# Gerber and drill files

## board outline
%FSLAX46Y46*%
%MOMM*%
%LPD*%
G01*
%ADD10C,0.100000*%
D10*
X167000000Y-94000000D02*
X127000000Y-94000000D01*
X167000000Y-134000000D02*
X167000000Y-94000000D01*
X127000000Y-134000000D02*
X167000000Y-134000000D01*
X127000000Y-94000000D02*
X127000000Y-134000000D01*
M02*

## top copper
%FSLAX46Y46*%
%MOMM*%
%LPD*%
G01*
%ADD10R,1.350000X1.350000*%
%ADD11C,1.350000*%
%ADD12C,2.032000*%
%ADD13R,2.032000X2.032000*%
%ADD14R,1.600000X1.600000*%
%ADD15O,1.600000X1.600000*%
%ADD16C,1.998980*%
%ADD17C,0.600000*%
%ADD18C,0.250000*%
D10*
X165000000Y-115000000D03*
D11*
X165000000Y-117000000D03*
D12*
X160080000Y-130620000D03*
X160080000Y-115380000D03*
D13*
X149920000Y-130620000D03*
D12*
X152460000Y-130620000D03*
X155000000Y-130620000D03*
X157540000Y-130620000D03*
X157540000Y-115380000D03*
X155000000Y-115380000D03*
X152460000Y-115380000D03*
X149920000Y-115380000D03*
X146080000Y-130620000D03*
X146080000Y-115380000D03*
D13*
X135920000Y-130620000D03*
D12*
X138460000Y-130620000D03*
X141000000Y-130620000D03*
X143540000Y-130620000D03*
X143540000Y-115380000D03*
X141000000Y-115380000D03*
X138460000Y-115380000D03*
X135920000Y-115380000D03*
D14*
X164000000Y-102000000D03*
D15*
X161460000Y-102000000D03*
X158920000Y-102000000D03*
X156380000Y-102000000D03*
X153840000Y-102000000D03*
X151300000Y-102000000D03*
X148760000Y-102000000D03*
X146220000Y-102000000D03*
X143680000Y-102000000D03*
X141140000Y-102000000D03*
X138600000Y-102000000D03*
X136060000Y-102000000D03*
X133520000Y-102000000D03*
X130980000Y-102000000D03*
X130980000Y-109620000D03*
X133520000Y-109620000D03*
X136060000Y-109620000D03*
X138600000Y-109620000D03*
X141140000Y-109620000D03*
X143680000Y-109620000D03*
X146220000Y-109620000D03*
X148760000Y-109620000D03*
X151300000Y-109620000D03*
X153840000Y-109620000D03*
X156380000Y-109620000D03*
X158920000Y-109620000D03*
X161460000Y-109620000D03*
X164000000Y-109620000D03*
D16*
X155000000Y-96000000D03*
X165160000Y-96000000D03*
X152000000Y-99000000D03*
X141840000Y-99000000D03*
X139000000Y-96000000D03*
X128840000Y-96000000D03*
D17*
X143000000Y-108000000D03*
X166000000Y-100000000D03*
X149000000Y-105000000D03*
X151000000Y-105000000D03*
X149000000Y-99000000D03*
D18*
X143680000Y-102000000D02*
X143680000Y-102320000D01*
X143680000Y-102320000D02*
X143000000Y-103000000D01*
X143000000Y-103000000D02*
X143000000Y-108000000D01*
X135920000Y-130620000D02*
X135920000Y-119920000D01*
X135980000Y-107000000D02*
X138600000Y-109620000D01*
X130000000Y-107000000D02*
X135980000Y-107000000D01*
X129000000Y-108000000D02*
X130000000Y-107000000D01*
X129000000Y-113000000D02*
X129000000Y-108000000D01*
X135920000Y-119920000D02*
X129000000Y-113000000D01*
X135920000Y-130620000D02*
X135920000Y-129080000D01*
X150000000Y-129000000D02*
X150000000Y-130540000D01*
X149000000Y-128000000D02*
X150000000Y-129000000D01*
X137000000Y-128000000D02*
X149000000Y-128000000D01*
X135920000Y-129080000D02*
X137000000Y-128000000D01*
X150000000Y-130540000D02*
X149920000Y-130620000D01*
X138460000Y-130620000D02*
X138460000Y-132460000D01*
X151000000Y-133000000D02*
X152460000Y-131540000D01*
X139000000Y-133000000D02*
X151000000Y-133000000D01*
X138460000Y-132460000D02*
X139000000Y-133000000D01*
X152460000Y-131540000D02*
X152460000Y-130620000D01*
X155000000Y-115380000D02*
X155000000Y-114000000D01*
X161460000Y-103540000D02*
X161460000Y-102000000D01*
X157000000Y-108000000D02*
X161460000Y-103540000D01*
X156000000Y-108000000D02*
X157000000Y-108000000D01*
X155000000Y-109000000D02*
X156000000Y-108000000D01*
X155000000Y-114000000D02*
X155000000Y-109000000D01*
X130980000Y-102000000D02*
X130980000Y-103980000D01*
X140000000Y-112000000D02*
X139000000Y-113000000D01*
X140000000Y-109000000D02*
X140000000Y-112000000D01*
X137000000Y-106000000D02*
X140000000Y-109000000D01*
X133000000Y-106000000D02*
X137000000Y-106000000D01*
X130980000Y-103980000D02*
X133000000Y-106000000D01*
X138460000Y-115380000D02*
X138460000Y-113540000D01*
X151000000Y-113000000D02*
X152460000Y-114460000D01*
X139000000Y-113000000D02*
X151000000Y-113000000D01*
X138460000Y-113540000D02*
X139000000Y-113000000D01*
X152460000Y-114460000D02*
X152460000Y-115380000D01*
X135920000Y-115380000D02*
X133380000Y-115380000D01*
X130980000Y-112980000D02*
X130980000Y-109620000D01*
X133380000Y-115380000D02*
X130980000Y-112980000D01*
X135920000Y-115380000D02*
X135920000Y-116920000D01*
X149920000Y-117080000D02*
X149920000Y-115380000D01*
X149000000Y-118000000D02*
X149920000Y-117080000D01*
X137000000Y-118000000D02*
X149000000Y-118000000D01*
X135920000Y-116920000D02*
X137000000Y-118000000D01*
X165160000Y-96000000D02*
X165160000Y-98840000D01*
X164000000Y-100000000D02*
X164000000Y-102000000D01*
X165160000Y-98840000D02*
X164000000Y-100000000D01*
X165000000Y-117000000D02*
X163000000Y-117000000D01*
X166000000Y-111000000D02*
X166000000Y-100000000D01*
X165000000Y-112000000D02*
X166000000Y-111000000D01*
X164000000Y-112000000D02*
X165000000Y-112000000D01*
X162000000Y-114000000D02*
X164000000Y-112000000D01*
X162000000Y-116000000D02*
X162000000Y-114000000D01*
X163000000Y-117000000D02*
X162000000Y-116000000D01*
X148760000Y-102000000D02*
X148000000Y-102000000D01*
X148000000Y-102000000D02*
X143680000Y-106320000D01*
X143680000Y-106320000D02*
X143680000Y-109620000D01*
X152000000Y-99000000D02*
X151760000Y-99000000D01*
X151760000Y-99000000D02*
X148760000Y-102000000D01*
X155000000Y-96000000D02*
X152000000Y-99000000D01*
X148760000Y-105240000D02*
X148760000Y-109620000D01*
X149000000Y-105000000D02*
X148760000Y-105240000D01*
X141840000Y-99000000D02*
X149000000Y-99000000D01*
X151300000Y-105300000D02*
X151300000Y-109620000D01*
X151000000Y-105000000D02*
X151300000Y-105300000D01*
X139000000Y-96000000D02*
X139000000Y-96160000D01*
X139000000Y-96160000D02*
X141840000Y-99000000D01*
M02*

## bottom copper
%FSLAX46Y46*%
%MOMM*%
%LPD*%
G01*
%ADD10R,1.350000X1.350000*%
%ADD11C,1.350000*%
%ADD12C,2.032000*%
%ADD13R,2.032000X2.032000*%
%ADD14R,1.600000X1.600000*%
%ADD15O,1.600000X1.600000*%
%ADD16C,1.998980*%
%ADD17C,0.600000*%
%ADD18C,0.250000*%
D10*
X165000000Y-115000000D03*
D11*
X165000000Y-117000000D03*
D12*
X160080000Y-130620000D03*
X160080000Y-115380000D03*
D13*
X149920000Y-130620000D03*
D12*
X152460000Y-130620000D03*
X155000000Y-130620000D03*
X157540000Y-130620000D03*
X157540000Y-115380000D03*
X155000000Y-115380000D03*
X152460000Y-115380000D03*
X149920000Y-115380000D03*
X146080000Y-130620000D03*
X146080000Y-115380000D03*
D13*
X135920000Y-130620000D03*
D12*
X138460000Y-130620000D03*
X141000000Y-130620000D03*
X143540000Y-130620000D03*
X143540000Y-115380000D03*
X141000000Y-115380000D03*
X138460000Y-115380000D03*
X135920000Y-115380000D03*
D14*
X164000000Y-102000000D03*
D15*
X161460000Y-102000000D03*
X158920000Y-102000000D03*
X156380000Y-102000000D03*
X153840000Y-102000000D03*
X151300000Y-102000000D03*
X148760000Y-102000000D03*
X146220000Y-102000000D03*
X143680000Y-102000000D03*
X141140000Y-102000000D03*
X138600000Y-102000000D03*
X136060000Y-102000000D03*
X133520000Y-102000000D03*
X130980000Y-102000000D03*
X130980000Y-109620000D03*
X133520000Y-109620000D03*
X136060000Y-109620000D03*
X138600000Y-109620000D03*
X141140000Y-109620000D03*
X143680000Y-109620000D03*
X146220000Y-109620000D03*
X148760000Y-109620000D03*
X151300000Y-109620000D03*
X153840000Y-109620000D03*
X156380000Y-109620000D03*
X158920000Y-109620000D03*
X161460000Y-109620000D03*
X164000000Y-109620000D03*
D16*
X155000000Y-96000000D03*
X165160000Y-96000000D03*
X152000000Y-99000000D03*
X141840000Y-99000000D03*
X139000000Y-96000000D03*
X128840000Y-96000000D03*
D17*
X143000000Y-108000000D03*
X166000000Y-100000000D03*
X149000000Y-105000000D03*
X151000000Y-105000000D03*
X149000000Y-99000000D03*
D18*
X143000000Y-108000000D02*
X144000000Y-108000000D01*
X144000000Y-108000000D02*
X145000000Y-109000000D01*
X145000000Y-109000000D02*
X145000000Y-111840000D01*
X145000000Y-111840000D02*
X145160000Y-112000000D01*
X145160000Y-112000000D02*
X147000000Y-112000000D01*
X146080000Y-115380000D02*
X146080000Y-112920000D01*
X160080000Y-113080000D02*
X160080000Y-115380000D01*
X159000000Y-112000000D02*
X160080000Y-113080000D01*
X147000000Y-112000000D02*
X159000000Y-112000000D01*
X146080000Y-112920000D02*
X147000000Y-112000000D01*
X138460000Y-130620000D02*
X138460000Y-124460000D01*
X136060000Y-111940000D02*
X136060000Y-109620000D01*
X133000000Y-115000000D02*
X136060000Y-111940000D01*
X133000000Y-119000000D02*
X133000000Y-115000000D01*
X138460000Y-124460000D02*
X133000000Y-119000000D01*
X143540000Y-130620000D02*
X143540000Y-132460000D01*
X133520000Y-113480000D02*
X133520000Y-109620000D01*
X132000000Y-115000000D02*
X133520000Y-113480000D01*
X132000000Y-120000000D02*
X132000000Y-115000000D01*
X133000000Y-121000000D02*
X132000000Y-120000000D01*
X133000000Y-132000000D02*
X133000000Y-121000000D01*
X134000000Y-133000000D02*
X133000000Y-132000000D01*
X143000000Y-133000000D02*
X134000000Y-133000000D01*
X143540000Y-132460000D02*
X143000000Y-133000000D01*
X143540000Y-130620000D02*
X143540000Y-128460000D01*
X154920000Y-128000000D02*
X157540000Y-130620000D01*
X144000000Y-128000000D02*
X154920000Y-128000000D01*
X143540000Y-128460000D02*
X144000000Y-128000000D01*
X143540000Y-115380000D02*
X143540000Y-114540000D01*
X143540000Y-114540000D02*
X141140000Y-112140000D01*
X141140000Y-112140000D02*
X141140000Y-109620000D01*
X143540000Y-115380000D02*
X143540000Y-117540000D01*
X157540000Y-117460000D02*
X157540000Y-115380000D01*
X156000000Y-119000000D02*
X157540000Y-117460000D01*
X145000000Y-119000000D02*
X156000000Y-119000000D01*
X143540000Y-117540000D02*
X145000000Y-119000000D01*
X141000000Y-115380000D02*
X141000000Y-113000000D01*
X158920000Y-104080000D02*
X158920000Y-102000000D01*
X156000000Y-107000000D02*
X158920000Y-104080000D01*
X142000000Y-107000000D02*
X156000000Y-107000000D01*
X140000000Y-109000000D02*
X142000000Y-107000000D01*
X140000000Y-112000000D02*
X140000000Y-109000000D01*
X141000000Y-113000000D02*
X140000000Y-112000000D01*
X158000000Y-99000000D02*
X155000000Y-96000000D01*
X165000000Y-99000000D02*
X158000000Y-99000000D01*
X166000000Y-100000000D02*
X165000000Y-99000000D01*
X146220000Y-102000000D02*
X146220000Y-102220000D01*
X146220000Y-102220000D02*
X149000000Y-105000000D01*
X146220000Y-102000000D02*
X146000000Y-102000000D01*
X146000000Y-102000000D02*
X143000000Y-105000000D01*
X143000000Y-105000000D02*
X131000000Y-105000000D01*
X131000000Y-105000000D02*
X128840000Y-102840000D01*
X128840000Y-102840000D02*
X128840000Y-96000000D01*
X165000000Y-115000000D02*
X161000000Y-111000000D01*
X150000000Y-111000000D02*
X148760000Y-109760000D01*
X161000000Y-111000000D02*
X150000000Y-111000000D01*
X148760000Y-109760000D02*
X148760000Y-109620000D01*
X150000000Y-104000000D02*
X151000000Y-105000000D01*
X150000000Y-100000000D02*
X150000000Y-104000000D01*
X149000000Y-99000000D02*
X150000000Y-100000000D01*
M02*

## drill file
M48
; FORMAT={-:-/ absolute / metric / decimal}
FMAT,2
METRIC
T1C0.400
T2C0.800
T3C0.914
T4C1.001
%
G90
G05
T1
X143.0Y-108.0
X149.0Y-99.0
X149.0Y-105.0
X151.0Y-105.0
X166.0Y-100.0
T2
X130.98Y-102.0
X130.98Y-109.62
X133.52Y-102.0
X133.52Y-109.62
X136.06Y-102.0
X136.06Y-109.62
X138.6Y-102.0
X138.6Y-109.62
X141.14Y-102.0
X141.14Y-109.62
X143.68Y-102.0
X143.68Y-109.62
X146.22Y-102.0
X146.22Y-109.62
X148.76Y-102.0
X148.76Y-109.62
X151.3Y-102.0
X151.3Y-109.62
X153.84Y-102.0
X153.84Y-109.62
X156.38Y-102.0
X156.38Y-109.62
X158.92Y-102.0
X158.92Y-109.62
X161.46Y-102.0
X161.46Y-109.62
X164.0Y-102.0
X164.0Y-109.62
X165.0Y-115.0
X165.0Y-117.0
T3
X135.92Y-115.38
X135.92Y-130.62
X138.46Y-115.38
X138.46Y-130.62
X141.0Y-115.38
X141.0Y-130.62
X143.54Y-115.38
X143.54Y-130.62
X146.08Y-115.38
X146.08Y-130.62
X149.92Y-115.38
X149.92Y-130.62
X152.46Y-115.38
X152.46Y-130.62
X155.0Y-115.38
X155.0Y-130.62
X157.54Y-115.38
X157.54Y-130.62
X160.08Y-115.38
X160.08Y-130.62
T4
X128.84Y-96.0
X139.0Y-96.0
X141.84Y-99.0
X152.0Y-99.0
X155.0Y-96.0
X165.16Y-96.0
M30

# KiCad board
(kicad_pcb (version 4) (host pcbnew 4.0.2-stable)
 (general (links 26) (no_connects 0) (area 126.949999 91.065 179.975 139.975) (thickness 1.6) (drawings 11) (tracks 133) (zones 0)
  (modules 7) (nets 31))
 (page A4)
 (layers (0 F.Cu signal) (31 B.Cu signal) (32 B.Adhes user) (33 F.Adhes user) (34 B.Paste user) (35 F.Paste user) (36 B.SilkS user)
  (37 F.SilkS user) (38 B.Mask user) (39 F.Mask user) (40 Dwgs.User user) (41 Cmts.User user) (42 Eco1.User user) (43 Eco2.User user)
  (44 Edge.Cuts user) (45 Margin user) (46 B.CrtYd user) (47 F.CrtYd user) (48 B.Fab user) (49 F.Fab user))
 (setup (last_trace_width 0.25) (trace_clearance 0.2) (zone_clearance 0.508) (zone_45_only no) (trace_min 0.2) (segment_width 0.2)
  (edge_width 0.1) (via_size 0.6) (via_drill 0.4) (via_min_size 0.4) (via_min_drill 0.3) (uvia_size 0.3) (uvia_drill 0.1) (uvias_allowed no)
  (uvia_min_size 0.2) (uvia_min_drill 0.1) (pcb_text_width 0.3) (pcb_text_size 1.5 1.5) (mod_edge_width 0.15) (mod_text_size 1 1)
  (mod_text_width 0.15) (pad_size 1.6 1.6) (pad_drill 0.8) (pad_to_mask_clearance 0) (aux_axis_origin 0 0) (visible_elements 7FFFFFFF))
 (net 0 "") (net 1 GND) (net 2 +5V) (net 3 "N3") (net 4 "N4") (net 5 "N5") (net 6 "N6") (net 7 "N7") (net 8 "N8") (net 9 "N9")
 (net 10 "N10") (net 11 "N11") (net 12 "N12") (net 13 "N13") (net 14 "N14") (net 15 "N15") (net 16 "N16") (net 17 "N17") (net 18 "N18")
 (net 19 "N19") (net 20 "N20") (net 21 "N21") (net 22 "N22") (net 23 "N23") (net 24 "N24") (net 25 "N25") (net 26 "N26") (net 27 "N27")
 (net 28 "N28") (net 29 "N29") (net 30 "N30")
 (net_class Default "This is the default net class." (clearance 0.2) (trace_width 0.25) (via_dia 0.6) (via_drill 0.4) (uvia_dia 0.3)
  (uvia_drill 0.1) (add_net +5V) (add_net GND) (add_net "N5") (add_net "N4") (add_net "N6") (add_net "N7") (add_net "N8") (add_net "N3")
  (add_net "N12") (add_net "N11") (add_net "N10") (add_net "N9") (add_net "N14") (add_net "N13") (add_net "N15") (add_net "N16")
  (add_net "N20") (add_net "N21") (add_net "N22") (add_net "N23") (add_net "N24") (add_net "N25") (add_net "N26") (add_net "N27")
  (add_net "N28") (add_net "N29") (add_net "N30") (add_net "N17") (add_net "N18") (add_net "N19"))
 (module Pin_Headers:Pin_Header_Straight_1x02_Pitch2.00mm (layer F.Cu) (at 165 115)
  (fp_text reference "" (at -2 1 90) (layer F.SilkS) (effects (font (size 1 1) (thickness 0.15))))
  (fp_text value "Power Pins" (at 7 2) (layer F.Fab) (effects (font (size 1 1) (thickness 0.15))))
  (pad 1 thru_hole rect (at 0 0) (size 1.35 1.35) (drill 0.8) (layers *.Cu *.Mask) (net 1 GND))
  (pad 2 thru_hole circle (at 0 2) (size 1.35 1.35) (drill 0.8) (layers *.Cu *.Mask) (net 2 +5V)))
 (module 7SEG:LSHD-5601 (layer F.Cu) (at 155 123)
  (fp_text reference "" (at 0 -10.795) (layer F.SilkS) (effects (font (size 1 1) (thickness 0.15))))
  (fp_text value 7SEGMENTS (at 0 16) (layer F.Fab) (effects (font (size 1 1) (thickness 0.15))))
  (pad 5 thru_hole circle (at 5.08 7.62) (size 2.032 2.032) (drill 0.9144) (layers *.Cu *.Mask F.SilkS) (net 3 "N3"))
  (pad 10 thru_hole circle (at 5.08 -7.62) (size 2.032 2.032) (drill 0.9144) (layers *.Cu *.Mask F.SilkS) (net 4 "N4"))
  (pad 1 thru_hole rect (at -5.08 7.62) (size 2.032 2.032) (drill 0.9144) (layers *.Cu *.Mask F.SilkS) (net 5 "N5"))
  (pad 2 thru_hole circle (at -2.54 7.62) (size 2.032 2.032) (drill 0.9144) (layers *.Cu *.Mask F.SilkS) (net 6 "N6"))
  (pad 3 thru_hole circle (at 0 7.62) (size 2.032 2.032) (drill 0.9144) (layers *.Cu *.Mask F.SilkS) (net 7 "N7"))
  (pad 4 thru_hole circle (at 2.54 7.62) (size 2.032 2.032) (drill 0.9144) (layers *.Cu *.Mask F.SilkS) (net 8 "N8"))
  (pad 9 thru_hole circle (at 2.54 -7.62) (size 2.032 2.032) (drill 0.9144) (layers *.Cu *.Mask F.SilkS) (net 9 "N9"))
  (pad 8 thru_hole circle (at 0 -7.62) (size 2.032 2.032) (drill 0.9144) (layers *.Cu *.Mask F.SilkS) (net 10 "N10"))
  (pad 7 thru_hole circle (at -2.54 -7.62) (size 2.032 2.032) (drill 0.9144) (layers *.Cu *.Mask F.SilkS) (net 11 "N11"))
  (pad 6 thru_hole circle (at -5.08 -7.62) (size 2.032 2.032) (drill 0.9144) (layers *.Cu *.Mask F.SilkS) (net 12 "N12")))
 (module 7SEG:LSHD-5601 (layer F.Cu) (at 141 123)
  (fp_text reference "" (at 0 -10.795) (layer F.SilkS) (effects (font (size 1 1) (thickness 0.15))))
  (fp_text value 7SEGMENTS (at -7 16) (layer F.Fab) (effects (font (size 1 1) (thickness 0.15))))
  (pad 5 thru_hole circle (at 5.08 7.62) (size 2.032 2.032) (drill 0.9144) (layers *.Cu *.Mask F.SilkS) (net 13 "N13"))
  (pad 10 thru_hole circle (at 5.08 -7.62) (size 2.032 2.032) (drill 0.9144) (layers *.Cu *.Mask F.SilkS) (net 4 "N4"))
  (pad 1 thru_hole rect (at -5.08 7.62) (size 2.032 2.032) (drill 0.9144) (layers *.Cu *.Mask F.SilkS) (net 5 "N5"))
  (pad 2 thru_hole circle (at -2.54 7.62) (size 2.032 2.032) (drill 0.9144) (layers *.Cu *.Mask F.SilkS) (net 6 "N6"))
  (pad 3 thru_hole circle (at 0 7.62) (size 2.032 2.032) (drill 0.9144) (layers *.Cu *.Mask F.SilkS) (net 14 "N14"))
  (pad 4 thru_hole circle (at 2.54 7.62) (size 2.032 2.032) (drill 0.9144) (layers *.Cu *.Mask F.SilkS) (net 8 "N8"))
  (pad 9 thru_hole circle (at 2.54 -7.62) (size 2.032 2.032) (drill 0.9144) (layers *.Cu *.Mask F.SilkS) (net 9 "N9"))
  (pad 8 thru_hole circle (at 0 -7.62) (size 2.032 2.032) (drill 0.9144) (layers *.Cu *.Mask F.SilkS) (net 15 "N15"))
  (pad 7 thru_hole circle (at -2.54 -7.62) (size 2.032 2.032) (drill 0.9144) (layers *.Cu *.Mask F.SilkS) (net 11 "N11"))
  (pad 6 thru_hole circle (at -5.08 -7.62) (size 2.032 2.032) (drill 0.9144) (layers *.Cu *.Mask F.SilkS) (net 12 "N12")))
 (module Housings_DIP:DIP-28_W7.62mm (layer F.Cu) (at 164 102 270)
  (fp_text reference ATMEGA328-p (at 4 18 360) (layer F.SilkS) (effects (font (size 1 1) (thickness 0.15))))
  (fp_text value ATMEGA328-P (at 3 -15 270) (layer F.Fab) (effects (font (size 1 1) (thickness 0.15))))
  (pad 1 thru_hole rect (at 0 0 270) (size 1.6 1.6) (drill 0.8) (layers *.Cu *.Mask F.SilkS) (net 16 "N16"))
  (pad 2 thru_hole oval (at 0 2.54 270) (size 1.6 1.6) (drill 0.8) (layers *.Cu *.Mask F.SilkS) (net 10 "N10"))
  (pad 3 thru_hole oval (at 0 5.08 270) (size 1.6 1.6) (drill 0.8) (layers *.Cu *.Mask F.SilkS) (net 15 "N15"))
  (pad 4 thru_hole oval (at 0 7.62 270) (size 1.6 1.6) (drill 0.8) (layers *.Cu *.Mask F.SilkS) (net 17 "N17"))
  (pad 5 thru_hole oval (at 0 10.16 270) (size 1.6 1.6) (drill 0.8) (layers *.Cu *.Mask F.SilkS) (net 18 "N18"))
  (pad 6 thru_hole oval (at 0 12.7 270) (size 1.6 1.6) (drill 0.8) (layers *.Cu *.Mask F.SilkS) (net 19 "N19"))
  (pad 7 thru_hole oval (at 0 15.24 270) (size 1.6 1.6) (drill 0.8) (layers *.Cu *.Mask F.SilkS) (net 2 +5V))
  (pad 8 thru_hole oval (at 0 17.78 270) (size 1.6 1.6) (drill 0.8) (layers *.Cu *.Mask F.SilkS) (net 1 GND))
  (pad 9 thru_hole oval (at 0 20.32 270) (size 1.6 1.6) (drill 0.8) (layers *.Cu *.Mask F.SilkS) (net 4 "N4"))
  (pad 10 thru_hole oval (at 0 22.86 270) (size 1.6 1.6) (drill 0.8) (layers *.Cu *.Mask F.SilkS) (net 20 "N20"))
  (pad 11 thru_hole oval (at 0 25.4 270) (size 1.6 1.6) (drill 0.8) (layers *.Cu *.Mask F.SilkS) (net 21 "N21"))
  (pad 12 thru_hole oval (at 0 27.94 270) (size 1.6 1.6) (drill 0.8) (layers *.Cu *.Mask F.SilkS) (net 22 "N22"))
  (pad 13 thru_hole oval (at 0 30.48 270) (size 1.6 1.6) (drill 0.8) (layers *.Cu *.Mask F.SilkS) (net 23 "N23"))
  (pad 14 thru_hole oval (at 0 33.02 270) (size 1.6 1.6) (drill 0.8) (layers *.Cu *.Mask F.SilkS) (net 11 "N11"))
  (pad 15 thru_hole oval (at 7.62 33.02 270) (size 1.6 1.6) (drill 0.8) (layers *.Cu *.Mask F.SilkS) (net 12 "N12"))
  (pad 16 thru_hole oval (at 7.62 30.48 270) (size 1.6 1.6) (drill 0.8) (layers *.Cu *.Mask F.SilkS) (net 8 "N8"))
  (pad 17 thru_hole oval (at 7.62 27.94 270) (size 1.6 1.6) (drill 0.8) (layers *.Cu *.Mask F.SilkS) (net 6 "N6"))
  (pad 18 thru_hole oval (at 7.62 25.4 270) (size 1.6 1.6) (drill 0.8) (layers *.Cu *.Mask F.SilkS) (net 5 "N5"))
  (pad 19 thru_hole oval (at 7.62 22.86 270) (size 1.6 1.6) (drill 0.8) (layers *.Cu *.Mask F.SilkS) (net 9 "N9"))
  (pad 20 thru_hole oval (at 7.62 20.32 270) (size 1.6 1.6) (drill 0.8) (layers *.Cu *.Mask F.SilkS) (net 2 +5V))
  (pad 21 thru_hole oval (at 7.62 17.78 270) (size 1.6 1.6) (drill 0.8) (layers *.Cu *.Mask F.SilkS) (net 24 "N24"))
  (pad 22 thru_hole oval (at 7.62 15.24 270) (size 1.6 1.6) (drill 0.8) (layers *.Cu *.Mask F.SilkS) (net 1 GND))
  (pad 23 thru_hole oval (at 7.62 12.7 270) (size 1.6 1.6) (drill 0.8) (layers *.Cu *.Mask F.SilkS) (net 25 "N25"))
  (pad 24 thru_hole oval (at 7.62 10.16 270) (size 1.6 1.6) (drill 0.8) (layers *.Cu *.Mask F.SilkS) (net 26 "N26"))
  (pad 25 thru_hole oval (at 7.62 7.62 270) (size 1.6 1.6) (drill 0.8) (layers *.Cu *.Mask F.SilkS) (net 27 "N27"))
  (pad 26 thru_hole oval (at 7.62 5.08 270) (size 1.6 1.6) (drill 0.8) (layers *.Cu *.Mask F.SilkS) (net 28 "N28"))
  (pad 27 thru_hole oval (at 7.62 2.54 270) (size 1.6 1.6) (drill 0.8) (layers *.Cu *.Mask F.SilkS) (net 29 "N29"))
  (pad 28 thru_hole oval (at 7.62 0 270) (size 1.6 1.6) (drill 0.8) (layers *.Cu *.Mask F.SilkS) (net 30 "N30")))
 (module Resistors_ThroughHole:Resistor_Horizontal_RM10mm (layer F.Cu) (at 155 96)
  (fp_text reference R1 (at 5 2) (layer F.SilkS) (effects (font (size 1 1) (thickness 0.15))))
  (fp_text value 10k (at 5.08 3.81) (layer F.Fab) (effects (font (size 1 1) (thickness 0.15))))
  (pad 1 thru_hole circle (at 0 0) (size 1.99898 1.99898) (drill 1.00076) (layers *.Cu *.SilkS *.Mask) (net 2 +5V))
  (pad 2 thru_hole circle (at 10.16 0) (size 1.99898 1.99898) (drill 1.00076) (layers *.Cu *.SilkS *.Mask) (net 16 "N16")))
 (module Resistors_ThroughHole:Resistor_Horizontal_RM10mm (layer F.Cu) (at 152 99 180)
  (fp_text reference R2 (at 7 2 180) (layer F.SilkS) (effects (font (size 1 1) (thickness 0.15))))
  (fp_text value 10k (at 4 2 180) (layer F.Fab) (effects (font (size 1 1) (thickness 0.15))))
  (pad 1 thru_hole circle (at 0 0 180) (size 1.99898 1.99898) (drill 1.00076) (layers *.Cu *.SilkS *.Mask) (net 2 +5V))
  (pad 2 thru_hole circle (at 10.16 0 180) (size 1.99898 1.99898) (drill 1.00076) (layers *.Cu *.SilkS *.Mask) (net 25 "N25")))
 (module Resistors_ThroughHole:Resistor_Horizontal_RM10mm (layer F.Cu) (at 139 96 180)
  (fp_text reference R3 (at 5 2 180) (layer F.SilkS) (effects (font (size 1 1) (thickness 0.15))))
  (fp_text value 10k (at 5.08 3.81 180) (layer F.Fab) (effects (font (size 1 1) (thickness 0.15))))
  (pad 1 thru_hole circle (at 0 0 180) (size 1.99898 1.99898) (drill 1.00076) (layers *.Cu *.SilkS *.Mask) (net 25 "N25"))
  (pad 2 thru_hole circle (at 10.16 0 180) (size 1.99898 1.99898) (drill 1.00076) (layers *.Cu *.SilkS *.Mask) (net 1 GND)))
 (gr_line (start 167 94) (end 127 94) (angle 90) (layer Edge.Cuts) (width 0.1))
 (gr_line (start 167 134) (end 167 94) (angle 90) (layer Edge.Cuts) (width 0.1))
 (gr_line (start 127 134) (end 167 134) (angle 90) (layer Edge.Cuts) (width 0.1))
 (gr_line (start 127 94) (end 127 134) (angle 90) (layer Edge.Cuts) (width 0.1))
 (segment (start 143.68 102) (end 143.68 102.32) (width 0.25) (layer F.Cu) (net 4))
 (segment (start 143.68 102.32) (end 143 103) (width 0.25) (layer F.Cu) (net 4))
 (segment (start 143 103) (end 143 108) (width 0.25) (layer F.Cu) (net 4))
 (via (at 143 108) (size 0.6) (drill 0.4) (layers F.Cu B.Cu) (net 4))
 (segment (start 143 108) (end 144 108) (width 0.25) (layer B.Cu) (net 4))
 (segment (start 144 108) (end 145 109) (width 0.25) (layer B.Cu) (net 4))
 (segment (start 145 109) (end 145 111.84) (width 0.25) (layer B.Cu) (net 4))
 (segment (start 145 111.84) (end 145.16 112) (width 0.25) (layer B.Cu) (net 4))
 (segment (start 145.16 112) (end 147 112) (width 0.25) (layer B.Cu) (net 4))
 (segment (start 146.08 115.38) (end 146.08 112.92) (width 0.25) (layer B.Cu) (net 4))
 (segment (start 160.08 113.08) (end 160.08 115.38) (width 0.25) (layer B.Cu) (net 4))
 (segment (start 159 112) (end 160.08 113.08) (width 0.25) (layer B.Cu) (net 4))
 (segment (start 147 112) (end 159 112) (width 0.25) (layer B.Cu) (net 4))
 (segment (start 146.08 112.92) (end 147 112) (width 0.25) (layer B.Cu) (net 4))
 (segment (start 135.92 130.62) (end 135.92 119.92) (width 0.25) (layer F.Cu) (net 5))
 (segment (start 135.98 107) (end 138.6 109.62) (width 0.25) (layer F.Cu) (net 5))
 (segment (start 130 107) (end 135.98 107) (width 0.25) (layer F.Cu) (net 5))
 (segment (start 129 108) (end 130 107) (width 0.25) (layer F.Cu) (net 5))
 (segment (start 129 113) (end 129 108) (width 0.25) (layer F.Cu) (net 5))
 (segment (start 135.92 119.92) (end 129 113) (width 0.25) (layer F.Cu) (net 5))
 (segment (start 135.92 130.62) (end 135.92 129.08) (width 0.25) (layer F.Cu) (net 5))
 (segment (start 150 129) (end 150 130.54) (width 0.25) (layer F.Cu) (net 5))
 (segment (start 149 128) (end 150 129) (width 0.25) (layer F.Cu) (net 5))
 (segment (start 137 128) (end 149 128) (width 0.25) (layer F.Cu) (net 5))
 (segment (start 135.92 129.08) (end 137 128) (width 0.25) (layer F.Cu) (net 5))
 (segment (start 150 130.54) (end 149.92 130.62) (width 0.25) (layer F.Cu) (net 5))
 (segment (start 138.46 130.62) (end 138.46 124.46) (width 0.25) (layer B.Cu) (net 6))
 (segment (start 136.06 111.94) (end 136.06 109.62) (width 0.25) (layer B.Cu) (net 6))
 (segment (start 133 115) (end 136.06 111.94) (width 0.25) (layer B.Cu) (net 6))
 (segment (start 133 119) (end 133 115) (width 0.25) (layer B.Cu) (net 6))
 (segment (start 138.46 124.46) (end 133 119) (width 0.25) (layer B.Cu) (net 6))
 (segment (start 138.46 130.62) (end 138.46 132.46) (width 0.25) (layer F.Cu) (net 6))
 (segment (start 151 133) (end 152.46 131.54) (width 0.25) (layer F.Cu) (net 6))
 (segment (start 139 133) (end 151 133) (width 0.25) (layer F.Cu) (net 6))
 (segment (start 138.46 132.46) (end 139 133) (width 0.25) (layer F.Cu) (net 6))
 (segment (start 152.46 131.54) (end 152.46 130.62) (width 0.25) (layer F.Cu) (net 6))
 (segment (start 143.54 130.62) (end 143.54 132.46) (width 0.25) (layer B.Cu) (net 8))
 (segment (start 133.52 113.48) (end 133.52 109.62) (width 0.25) (layer B.Cu) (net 8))
 (segment (start 132 115) (end 133.52 113.48) (width 0.25) (layer B.Cu) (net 8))
 (segment (start 132 120) (end 132 115) (width 0.25) (layer B.Cu) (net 8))
 (segment (start 133 121) (end 132 120) (width 0.25) (layer B.Cu) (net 8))
 (segment (start 133 132) (end 133 121) (width 0.25) (layer B.Cu) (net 8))
 (segment (start 134 133) (end 133 132) (width 0.25) (layer B.Cu) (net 8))
 (segment (start 143 133) (end 134 133) (width 0.25) (layer B.Cu) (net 8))
 (segment (start 143.54 132.46) (end 143 133) (width 0.25) (layer B.Cu) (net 8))
 (segment (start 143.54 130.62) (end 143.54 128.46) (width 0.25) (layer B.Cu) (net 8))
 (segment (start 154.92 128) (end 157.54 130.62) (width 0.25) (layer B.Cu) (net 8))
 (segment (start 144 128) (end 154.92 128) (width 0.25) (layer B.Cu) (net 8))
 (segment (start 143.54 128.46) (end 144 128) (width 0.25) (layer B.Cu) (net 8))
 (segment (start 143.54 115.38) (end 143.54 114.54) (width 0.25) (layer B.Cu) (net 9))
 (segment (start 143.54 114.54) (end 141.14 112.14) (width 0.25) (layer B.Cu) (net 9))
 (segment (start 141.14 112.14) (end 141.14 109.62) (width 0.25) (layer B.Cu) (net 9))
 (segment (start 143.54 115.38) (end 143.54 117.54) (width 0.25) (layer B.Cu) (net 9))
 (segment (start 157.54 117.46) (end 157.54 115.38) (width 0.25) (layer B.Cu) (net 9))
 (segment (start 156 119) (end 157.54 117.46) (width 0.25) (layer B.Cu) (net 9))
 (segment (start 145 119) (end 156 119) (width 0.25) (layer B.Cu) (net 9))
 (segment (start 143.54 117.54) (end 145 119) (width 0.25) (layer B.Cu) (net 9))
 (segment (start 155 115.38) (end 155 114) (width 0.25) (layer F.Cu) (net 10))
 (segment (start 161.46 103.54) (end 161.46 102) (width 0.25) (layer F.Cu) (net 10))
 (segment (start 157 108) (end 161.46 103.54) (width 0.25) (layer F.Cu) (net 10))
 (segment (start 156 108) (end 157 108) (width 0.25) (layer F.Cu) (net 10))
 (segment (start 155 109) (end 156 108) (width 0.25) (layer F.Cu) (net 10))
 (segment (start 155 114) (end 155 109) (width 0.25) (layer F.Cu) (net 10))
 (segment (start 130.98 102) (end 130.98 103.98) (width 0.25) (layer F.Cu) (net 11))
 (segment (start 140 112) (end 139 113) (width 0.25) (layer F.Cu) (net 11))
 (segment (start 140 109) (end 140 112) (width 0.25) (layer F.Cu) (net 11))
 (segment (start 137 106) (end 140 109) (width 0.25) (layer F.Cu) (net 11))
 (segment (start 133 106) (end 137 106) (width 0.25) (layer F.Cu) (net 11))
 (segment (start 130.98 103.98) (end 133 106) (width 0.25) (layer F.Cu) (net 11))
 (segment (start 138.46 115.38) (end 138.46 113.54) (width 0.25) (layer F.Cu) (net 11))
 (segment (start 151 113) (end 152.46 114.46) (width 0.25) (layer F.Cu) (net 11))
 (segment (start 139 113) (end 151 113) (width 0.25) (layer F.Cu) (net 11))
 (segment (start 138.46 113.54) (end 139 113) (width 0.25) (layer F.Cu) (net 11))
 (segment (start 152.46 114.46) (end 152.46 115.38) (width 0.25) (layer F.Cu) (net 11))
 (segment (start 135.92 115.38) (end 133.38 115.38) (width 0.25) (layer F.Cu) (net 12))
 (segment (start 130.98 112.98) (end 130.98 109.62) (width 0.25) (layer F.Cu) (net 12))
 (segment (start 133.38 115.38) (end 130.98 112.98) (width 0.25) (layer F.Cu) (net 12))
 (segment (start 135.92 115.38) (end 135.92 116.92) (width 0.25) (layer F.Cu) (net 12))
 (segment (start 149.92 117.08) (end 149.92 115.38) (width 0.25) (layer F.Cu) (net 12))
 (segment (start 149 118) (end 149.92 117.08) (width 0.25) (layer F.Cu) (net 12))
 (segment (start 137 118) (end 149 118) (width 0.25) (layer F.Cu) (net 12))
 (segment (start 135.92 116.92) (end 137 118) (width 0.25) (layer F.Cu) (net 12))
 (segment (start 141 115.38) (end 141 113) (width 0.25) (layer B.Cu) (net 15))
 (segment (start 158.92 104.08) (end 158.92 102) (width 0.25) (layer B.Cu) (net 15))
 (segment (start 156 107) (end 158.92 104.08) (width 0.25) (layer B.Cu) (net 15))
 (segment (start 142 107) (end 156 107) (width 0.25) (layer B.Cu) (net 15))
 (segment (start 140 109) (end 142 107) (width 0.25) (layer B.Cu) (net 15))
 (segment (start 140 112) (end 140 109) (width 0.25) (layer B.Cu) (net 15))
 (segment (start 141 113) (end 140 112) (width 0.25) (layer B.Cu) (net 15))
 (segment (start 165.16 96) (end 165.16 98.84) (width 0.25) (layer F.Cu) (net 16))
 (segment (start 164 100) (end 164 102) (width 0.25) (layer F.Cu) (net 16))
 (segment (start 165.16 98.84) (end 164 100) (width 0.25) (layer F.Cu) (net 16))
 (segment (start 165 117) (end 163 117) (width 0.25) (layer F.Cu) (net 2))
 (segment (start 158 99) (end 155 96) (width 0.25) (layer B.Cu) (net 2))
 (segment (start 165 99) (end 158 99) (width 0.25) (layer B.Cu) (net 2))
 (segment (start 166 100) (end 165 99) (width 0.25) (layer B.Cu) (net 2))
 (via (at 166 100) (size 0.6) (drill 0.4) (layers F.Cu B.Cu) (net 2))
 (segment (start 166 111) (end 166 100) (width 0.25) (layer F.Cu) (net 2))
 (segment (start 165 112) (end 166 111) (width 0.25) (layer F.Cu) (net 2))
 (segment (start 164 112) (end 165 112) (width 0.25) (layer F.Cu) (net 2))
 (segment (start 162 114) (end 164 112) (width 0.25) (layer F.Cu) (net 2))
 (segment (start 162 116) (end 162 114) (width 0.25) (layer F.Cu) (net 2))
 (segment (start 163 117) (end 162 116) (width 0.25) (layer F.Cu) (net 2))
 (segment (start 148.76 102) (end 148 102) (width 0.25) (layer F.Cu) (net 2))
 (segment (start 148 102) (end 143.68 106.32) (width 0.25) (layer F.Cu) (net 2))
 (segment (start 143.68 106.32) (end 143.68 109.62) (width 0.25) (layer F.Cu) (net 2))
 (segment (start 152 99) (end 151.76 99) (width 0.25) (layer F.Cu) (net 2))
 (segment (start 151.76 99) (end 148.76 102) (width 0.25) (layer F.Cu) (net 2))
 (segment (start 155 96) (end 152 99) (width 0.25) (layer F.Cu) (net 2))
 (segment (start 146.22 102) (end 146.22 102.22) (width 0.25) (layer B.Cu) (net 1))
 (segment (start 146.22 102.22) (end 149 105) (width 0.25) (layer B.Cu) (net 1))
 (segment (start 148.76 105.24) (end 148.76 109.62) (width 0.25) (layer F.Cu) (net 1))
 (segment (start 149 105) (end 148.76 105.24) (width 0.25) (layer F.Cu) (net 1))
 (via (at 149 105) (size 0.6) (drill 0.4) (layers F.Cu B.Cu) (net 1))
 (segment (start 146.22 102) (end 146 102) (width 0.25) (layer B.Cu) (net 1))
 (segment (start 146 102) (end 143 105) (width 0.25) (layer B.Cu) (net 1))
 (segment (start 143 105) (end 131 105) (width 0.25) (layer B.Cu) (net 1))
 (segment (start 131 105) (end 128.84 102.84) (width 0.25) (layer B.Cu) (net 1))
 (segment (start 128.84 102.84) (end 128.84 96) (width 0.25) (layer B.Cu) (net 1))
 (segment (start 165 115) (end 161 111) (width 0.25) (layer B.Cu) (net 1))
 (segment (start 150 111) (end 148.76 109.76) (width 0.25) (layer B.Cu) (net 1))
 (segment (start 161 111) (end 150 111) (width 0.25) (layer B.Cu) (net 1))
 (segment (start 148.76 109.76) (end 148.76 109.62) (width 0.25) (layer B.Cu) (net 1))
 (segment (start 141.84 99) (end 149 99) (width 0.25) (layer F.Cu) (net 25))
 (segment (start 151.3 105.3) (end 151.3 109.62) (width 0.25) (layer F.Cu) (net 25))
 (segment (start 151 105) (end 151.3 105.3) (width 0.25) (layer F.Cu) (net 25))
 (via (at 151 105) (size 0.6) (drill 0.4) (layers F.Cu B.Cu) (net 25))
 (segment (start 150 104) (end 151 105) (width 0.25) (layer B.Cu) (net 25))
 (segment (start 150 100) (end 150 104) (width 0.25) (layer B.Cu) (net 25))
 (segment (start 149 99) (end 150 100) (width 0.25) (layer B.Cu) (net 25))
 (via (at 149 99) (size 0.6) (drill 0.4) (layers F.Cu B.Cu) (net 25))
 (segment (start 139 96) (end 139 96.16) (width 0.25) (layer F.Cu) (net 25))
 (segment (start 139 96.16) (end 141.84 99) (width 0.25) (layer F.Cu) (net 25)))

